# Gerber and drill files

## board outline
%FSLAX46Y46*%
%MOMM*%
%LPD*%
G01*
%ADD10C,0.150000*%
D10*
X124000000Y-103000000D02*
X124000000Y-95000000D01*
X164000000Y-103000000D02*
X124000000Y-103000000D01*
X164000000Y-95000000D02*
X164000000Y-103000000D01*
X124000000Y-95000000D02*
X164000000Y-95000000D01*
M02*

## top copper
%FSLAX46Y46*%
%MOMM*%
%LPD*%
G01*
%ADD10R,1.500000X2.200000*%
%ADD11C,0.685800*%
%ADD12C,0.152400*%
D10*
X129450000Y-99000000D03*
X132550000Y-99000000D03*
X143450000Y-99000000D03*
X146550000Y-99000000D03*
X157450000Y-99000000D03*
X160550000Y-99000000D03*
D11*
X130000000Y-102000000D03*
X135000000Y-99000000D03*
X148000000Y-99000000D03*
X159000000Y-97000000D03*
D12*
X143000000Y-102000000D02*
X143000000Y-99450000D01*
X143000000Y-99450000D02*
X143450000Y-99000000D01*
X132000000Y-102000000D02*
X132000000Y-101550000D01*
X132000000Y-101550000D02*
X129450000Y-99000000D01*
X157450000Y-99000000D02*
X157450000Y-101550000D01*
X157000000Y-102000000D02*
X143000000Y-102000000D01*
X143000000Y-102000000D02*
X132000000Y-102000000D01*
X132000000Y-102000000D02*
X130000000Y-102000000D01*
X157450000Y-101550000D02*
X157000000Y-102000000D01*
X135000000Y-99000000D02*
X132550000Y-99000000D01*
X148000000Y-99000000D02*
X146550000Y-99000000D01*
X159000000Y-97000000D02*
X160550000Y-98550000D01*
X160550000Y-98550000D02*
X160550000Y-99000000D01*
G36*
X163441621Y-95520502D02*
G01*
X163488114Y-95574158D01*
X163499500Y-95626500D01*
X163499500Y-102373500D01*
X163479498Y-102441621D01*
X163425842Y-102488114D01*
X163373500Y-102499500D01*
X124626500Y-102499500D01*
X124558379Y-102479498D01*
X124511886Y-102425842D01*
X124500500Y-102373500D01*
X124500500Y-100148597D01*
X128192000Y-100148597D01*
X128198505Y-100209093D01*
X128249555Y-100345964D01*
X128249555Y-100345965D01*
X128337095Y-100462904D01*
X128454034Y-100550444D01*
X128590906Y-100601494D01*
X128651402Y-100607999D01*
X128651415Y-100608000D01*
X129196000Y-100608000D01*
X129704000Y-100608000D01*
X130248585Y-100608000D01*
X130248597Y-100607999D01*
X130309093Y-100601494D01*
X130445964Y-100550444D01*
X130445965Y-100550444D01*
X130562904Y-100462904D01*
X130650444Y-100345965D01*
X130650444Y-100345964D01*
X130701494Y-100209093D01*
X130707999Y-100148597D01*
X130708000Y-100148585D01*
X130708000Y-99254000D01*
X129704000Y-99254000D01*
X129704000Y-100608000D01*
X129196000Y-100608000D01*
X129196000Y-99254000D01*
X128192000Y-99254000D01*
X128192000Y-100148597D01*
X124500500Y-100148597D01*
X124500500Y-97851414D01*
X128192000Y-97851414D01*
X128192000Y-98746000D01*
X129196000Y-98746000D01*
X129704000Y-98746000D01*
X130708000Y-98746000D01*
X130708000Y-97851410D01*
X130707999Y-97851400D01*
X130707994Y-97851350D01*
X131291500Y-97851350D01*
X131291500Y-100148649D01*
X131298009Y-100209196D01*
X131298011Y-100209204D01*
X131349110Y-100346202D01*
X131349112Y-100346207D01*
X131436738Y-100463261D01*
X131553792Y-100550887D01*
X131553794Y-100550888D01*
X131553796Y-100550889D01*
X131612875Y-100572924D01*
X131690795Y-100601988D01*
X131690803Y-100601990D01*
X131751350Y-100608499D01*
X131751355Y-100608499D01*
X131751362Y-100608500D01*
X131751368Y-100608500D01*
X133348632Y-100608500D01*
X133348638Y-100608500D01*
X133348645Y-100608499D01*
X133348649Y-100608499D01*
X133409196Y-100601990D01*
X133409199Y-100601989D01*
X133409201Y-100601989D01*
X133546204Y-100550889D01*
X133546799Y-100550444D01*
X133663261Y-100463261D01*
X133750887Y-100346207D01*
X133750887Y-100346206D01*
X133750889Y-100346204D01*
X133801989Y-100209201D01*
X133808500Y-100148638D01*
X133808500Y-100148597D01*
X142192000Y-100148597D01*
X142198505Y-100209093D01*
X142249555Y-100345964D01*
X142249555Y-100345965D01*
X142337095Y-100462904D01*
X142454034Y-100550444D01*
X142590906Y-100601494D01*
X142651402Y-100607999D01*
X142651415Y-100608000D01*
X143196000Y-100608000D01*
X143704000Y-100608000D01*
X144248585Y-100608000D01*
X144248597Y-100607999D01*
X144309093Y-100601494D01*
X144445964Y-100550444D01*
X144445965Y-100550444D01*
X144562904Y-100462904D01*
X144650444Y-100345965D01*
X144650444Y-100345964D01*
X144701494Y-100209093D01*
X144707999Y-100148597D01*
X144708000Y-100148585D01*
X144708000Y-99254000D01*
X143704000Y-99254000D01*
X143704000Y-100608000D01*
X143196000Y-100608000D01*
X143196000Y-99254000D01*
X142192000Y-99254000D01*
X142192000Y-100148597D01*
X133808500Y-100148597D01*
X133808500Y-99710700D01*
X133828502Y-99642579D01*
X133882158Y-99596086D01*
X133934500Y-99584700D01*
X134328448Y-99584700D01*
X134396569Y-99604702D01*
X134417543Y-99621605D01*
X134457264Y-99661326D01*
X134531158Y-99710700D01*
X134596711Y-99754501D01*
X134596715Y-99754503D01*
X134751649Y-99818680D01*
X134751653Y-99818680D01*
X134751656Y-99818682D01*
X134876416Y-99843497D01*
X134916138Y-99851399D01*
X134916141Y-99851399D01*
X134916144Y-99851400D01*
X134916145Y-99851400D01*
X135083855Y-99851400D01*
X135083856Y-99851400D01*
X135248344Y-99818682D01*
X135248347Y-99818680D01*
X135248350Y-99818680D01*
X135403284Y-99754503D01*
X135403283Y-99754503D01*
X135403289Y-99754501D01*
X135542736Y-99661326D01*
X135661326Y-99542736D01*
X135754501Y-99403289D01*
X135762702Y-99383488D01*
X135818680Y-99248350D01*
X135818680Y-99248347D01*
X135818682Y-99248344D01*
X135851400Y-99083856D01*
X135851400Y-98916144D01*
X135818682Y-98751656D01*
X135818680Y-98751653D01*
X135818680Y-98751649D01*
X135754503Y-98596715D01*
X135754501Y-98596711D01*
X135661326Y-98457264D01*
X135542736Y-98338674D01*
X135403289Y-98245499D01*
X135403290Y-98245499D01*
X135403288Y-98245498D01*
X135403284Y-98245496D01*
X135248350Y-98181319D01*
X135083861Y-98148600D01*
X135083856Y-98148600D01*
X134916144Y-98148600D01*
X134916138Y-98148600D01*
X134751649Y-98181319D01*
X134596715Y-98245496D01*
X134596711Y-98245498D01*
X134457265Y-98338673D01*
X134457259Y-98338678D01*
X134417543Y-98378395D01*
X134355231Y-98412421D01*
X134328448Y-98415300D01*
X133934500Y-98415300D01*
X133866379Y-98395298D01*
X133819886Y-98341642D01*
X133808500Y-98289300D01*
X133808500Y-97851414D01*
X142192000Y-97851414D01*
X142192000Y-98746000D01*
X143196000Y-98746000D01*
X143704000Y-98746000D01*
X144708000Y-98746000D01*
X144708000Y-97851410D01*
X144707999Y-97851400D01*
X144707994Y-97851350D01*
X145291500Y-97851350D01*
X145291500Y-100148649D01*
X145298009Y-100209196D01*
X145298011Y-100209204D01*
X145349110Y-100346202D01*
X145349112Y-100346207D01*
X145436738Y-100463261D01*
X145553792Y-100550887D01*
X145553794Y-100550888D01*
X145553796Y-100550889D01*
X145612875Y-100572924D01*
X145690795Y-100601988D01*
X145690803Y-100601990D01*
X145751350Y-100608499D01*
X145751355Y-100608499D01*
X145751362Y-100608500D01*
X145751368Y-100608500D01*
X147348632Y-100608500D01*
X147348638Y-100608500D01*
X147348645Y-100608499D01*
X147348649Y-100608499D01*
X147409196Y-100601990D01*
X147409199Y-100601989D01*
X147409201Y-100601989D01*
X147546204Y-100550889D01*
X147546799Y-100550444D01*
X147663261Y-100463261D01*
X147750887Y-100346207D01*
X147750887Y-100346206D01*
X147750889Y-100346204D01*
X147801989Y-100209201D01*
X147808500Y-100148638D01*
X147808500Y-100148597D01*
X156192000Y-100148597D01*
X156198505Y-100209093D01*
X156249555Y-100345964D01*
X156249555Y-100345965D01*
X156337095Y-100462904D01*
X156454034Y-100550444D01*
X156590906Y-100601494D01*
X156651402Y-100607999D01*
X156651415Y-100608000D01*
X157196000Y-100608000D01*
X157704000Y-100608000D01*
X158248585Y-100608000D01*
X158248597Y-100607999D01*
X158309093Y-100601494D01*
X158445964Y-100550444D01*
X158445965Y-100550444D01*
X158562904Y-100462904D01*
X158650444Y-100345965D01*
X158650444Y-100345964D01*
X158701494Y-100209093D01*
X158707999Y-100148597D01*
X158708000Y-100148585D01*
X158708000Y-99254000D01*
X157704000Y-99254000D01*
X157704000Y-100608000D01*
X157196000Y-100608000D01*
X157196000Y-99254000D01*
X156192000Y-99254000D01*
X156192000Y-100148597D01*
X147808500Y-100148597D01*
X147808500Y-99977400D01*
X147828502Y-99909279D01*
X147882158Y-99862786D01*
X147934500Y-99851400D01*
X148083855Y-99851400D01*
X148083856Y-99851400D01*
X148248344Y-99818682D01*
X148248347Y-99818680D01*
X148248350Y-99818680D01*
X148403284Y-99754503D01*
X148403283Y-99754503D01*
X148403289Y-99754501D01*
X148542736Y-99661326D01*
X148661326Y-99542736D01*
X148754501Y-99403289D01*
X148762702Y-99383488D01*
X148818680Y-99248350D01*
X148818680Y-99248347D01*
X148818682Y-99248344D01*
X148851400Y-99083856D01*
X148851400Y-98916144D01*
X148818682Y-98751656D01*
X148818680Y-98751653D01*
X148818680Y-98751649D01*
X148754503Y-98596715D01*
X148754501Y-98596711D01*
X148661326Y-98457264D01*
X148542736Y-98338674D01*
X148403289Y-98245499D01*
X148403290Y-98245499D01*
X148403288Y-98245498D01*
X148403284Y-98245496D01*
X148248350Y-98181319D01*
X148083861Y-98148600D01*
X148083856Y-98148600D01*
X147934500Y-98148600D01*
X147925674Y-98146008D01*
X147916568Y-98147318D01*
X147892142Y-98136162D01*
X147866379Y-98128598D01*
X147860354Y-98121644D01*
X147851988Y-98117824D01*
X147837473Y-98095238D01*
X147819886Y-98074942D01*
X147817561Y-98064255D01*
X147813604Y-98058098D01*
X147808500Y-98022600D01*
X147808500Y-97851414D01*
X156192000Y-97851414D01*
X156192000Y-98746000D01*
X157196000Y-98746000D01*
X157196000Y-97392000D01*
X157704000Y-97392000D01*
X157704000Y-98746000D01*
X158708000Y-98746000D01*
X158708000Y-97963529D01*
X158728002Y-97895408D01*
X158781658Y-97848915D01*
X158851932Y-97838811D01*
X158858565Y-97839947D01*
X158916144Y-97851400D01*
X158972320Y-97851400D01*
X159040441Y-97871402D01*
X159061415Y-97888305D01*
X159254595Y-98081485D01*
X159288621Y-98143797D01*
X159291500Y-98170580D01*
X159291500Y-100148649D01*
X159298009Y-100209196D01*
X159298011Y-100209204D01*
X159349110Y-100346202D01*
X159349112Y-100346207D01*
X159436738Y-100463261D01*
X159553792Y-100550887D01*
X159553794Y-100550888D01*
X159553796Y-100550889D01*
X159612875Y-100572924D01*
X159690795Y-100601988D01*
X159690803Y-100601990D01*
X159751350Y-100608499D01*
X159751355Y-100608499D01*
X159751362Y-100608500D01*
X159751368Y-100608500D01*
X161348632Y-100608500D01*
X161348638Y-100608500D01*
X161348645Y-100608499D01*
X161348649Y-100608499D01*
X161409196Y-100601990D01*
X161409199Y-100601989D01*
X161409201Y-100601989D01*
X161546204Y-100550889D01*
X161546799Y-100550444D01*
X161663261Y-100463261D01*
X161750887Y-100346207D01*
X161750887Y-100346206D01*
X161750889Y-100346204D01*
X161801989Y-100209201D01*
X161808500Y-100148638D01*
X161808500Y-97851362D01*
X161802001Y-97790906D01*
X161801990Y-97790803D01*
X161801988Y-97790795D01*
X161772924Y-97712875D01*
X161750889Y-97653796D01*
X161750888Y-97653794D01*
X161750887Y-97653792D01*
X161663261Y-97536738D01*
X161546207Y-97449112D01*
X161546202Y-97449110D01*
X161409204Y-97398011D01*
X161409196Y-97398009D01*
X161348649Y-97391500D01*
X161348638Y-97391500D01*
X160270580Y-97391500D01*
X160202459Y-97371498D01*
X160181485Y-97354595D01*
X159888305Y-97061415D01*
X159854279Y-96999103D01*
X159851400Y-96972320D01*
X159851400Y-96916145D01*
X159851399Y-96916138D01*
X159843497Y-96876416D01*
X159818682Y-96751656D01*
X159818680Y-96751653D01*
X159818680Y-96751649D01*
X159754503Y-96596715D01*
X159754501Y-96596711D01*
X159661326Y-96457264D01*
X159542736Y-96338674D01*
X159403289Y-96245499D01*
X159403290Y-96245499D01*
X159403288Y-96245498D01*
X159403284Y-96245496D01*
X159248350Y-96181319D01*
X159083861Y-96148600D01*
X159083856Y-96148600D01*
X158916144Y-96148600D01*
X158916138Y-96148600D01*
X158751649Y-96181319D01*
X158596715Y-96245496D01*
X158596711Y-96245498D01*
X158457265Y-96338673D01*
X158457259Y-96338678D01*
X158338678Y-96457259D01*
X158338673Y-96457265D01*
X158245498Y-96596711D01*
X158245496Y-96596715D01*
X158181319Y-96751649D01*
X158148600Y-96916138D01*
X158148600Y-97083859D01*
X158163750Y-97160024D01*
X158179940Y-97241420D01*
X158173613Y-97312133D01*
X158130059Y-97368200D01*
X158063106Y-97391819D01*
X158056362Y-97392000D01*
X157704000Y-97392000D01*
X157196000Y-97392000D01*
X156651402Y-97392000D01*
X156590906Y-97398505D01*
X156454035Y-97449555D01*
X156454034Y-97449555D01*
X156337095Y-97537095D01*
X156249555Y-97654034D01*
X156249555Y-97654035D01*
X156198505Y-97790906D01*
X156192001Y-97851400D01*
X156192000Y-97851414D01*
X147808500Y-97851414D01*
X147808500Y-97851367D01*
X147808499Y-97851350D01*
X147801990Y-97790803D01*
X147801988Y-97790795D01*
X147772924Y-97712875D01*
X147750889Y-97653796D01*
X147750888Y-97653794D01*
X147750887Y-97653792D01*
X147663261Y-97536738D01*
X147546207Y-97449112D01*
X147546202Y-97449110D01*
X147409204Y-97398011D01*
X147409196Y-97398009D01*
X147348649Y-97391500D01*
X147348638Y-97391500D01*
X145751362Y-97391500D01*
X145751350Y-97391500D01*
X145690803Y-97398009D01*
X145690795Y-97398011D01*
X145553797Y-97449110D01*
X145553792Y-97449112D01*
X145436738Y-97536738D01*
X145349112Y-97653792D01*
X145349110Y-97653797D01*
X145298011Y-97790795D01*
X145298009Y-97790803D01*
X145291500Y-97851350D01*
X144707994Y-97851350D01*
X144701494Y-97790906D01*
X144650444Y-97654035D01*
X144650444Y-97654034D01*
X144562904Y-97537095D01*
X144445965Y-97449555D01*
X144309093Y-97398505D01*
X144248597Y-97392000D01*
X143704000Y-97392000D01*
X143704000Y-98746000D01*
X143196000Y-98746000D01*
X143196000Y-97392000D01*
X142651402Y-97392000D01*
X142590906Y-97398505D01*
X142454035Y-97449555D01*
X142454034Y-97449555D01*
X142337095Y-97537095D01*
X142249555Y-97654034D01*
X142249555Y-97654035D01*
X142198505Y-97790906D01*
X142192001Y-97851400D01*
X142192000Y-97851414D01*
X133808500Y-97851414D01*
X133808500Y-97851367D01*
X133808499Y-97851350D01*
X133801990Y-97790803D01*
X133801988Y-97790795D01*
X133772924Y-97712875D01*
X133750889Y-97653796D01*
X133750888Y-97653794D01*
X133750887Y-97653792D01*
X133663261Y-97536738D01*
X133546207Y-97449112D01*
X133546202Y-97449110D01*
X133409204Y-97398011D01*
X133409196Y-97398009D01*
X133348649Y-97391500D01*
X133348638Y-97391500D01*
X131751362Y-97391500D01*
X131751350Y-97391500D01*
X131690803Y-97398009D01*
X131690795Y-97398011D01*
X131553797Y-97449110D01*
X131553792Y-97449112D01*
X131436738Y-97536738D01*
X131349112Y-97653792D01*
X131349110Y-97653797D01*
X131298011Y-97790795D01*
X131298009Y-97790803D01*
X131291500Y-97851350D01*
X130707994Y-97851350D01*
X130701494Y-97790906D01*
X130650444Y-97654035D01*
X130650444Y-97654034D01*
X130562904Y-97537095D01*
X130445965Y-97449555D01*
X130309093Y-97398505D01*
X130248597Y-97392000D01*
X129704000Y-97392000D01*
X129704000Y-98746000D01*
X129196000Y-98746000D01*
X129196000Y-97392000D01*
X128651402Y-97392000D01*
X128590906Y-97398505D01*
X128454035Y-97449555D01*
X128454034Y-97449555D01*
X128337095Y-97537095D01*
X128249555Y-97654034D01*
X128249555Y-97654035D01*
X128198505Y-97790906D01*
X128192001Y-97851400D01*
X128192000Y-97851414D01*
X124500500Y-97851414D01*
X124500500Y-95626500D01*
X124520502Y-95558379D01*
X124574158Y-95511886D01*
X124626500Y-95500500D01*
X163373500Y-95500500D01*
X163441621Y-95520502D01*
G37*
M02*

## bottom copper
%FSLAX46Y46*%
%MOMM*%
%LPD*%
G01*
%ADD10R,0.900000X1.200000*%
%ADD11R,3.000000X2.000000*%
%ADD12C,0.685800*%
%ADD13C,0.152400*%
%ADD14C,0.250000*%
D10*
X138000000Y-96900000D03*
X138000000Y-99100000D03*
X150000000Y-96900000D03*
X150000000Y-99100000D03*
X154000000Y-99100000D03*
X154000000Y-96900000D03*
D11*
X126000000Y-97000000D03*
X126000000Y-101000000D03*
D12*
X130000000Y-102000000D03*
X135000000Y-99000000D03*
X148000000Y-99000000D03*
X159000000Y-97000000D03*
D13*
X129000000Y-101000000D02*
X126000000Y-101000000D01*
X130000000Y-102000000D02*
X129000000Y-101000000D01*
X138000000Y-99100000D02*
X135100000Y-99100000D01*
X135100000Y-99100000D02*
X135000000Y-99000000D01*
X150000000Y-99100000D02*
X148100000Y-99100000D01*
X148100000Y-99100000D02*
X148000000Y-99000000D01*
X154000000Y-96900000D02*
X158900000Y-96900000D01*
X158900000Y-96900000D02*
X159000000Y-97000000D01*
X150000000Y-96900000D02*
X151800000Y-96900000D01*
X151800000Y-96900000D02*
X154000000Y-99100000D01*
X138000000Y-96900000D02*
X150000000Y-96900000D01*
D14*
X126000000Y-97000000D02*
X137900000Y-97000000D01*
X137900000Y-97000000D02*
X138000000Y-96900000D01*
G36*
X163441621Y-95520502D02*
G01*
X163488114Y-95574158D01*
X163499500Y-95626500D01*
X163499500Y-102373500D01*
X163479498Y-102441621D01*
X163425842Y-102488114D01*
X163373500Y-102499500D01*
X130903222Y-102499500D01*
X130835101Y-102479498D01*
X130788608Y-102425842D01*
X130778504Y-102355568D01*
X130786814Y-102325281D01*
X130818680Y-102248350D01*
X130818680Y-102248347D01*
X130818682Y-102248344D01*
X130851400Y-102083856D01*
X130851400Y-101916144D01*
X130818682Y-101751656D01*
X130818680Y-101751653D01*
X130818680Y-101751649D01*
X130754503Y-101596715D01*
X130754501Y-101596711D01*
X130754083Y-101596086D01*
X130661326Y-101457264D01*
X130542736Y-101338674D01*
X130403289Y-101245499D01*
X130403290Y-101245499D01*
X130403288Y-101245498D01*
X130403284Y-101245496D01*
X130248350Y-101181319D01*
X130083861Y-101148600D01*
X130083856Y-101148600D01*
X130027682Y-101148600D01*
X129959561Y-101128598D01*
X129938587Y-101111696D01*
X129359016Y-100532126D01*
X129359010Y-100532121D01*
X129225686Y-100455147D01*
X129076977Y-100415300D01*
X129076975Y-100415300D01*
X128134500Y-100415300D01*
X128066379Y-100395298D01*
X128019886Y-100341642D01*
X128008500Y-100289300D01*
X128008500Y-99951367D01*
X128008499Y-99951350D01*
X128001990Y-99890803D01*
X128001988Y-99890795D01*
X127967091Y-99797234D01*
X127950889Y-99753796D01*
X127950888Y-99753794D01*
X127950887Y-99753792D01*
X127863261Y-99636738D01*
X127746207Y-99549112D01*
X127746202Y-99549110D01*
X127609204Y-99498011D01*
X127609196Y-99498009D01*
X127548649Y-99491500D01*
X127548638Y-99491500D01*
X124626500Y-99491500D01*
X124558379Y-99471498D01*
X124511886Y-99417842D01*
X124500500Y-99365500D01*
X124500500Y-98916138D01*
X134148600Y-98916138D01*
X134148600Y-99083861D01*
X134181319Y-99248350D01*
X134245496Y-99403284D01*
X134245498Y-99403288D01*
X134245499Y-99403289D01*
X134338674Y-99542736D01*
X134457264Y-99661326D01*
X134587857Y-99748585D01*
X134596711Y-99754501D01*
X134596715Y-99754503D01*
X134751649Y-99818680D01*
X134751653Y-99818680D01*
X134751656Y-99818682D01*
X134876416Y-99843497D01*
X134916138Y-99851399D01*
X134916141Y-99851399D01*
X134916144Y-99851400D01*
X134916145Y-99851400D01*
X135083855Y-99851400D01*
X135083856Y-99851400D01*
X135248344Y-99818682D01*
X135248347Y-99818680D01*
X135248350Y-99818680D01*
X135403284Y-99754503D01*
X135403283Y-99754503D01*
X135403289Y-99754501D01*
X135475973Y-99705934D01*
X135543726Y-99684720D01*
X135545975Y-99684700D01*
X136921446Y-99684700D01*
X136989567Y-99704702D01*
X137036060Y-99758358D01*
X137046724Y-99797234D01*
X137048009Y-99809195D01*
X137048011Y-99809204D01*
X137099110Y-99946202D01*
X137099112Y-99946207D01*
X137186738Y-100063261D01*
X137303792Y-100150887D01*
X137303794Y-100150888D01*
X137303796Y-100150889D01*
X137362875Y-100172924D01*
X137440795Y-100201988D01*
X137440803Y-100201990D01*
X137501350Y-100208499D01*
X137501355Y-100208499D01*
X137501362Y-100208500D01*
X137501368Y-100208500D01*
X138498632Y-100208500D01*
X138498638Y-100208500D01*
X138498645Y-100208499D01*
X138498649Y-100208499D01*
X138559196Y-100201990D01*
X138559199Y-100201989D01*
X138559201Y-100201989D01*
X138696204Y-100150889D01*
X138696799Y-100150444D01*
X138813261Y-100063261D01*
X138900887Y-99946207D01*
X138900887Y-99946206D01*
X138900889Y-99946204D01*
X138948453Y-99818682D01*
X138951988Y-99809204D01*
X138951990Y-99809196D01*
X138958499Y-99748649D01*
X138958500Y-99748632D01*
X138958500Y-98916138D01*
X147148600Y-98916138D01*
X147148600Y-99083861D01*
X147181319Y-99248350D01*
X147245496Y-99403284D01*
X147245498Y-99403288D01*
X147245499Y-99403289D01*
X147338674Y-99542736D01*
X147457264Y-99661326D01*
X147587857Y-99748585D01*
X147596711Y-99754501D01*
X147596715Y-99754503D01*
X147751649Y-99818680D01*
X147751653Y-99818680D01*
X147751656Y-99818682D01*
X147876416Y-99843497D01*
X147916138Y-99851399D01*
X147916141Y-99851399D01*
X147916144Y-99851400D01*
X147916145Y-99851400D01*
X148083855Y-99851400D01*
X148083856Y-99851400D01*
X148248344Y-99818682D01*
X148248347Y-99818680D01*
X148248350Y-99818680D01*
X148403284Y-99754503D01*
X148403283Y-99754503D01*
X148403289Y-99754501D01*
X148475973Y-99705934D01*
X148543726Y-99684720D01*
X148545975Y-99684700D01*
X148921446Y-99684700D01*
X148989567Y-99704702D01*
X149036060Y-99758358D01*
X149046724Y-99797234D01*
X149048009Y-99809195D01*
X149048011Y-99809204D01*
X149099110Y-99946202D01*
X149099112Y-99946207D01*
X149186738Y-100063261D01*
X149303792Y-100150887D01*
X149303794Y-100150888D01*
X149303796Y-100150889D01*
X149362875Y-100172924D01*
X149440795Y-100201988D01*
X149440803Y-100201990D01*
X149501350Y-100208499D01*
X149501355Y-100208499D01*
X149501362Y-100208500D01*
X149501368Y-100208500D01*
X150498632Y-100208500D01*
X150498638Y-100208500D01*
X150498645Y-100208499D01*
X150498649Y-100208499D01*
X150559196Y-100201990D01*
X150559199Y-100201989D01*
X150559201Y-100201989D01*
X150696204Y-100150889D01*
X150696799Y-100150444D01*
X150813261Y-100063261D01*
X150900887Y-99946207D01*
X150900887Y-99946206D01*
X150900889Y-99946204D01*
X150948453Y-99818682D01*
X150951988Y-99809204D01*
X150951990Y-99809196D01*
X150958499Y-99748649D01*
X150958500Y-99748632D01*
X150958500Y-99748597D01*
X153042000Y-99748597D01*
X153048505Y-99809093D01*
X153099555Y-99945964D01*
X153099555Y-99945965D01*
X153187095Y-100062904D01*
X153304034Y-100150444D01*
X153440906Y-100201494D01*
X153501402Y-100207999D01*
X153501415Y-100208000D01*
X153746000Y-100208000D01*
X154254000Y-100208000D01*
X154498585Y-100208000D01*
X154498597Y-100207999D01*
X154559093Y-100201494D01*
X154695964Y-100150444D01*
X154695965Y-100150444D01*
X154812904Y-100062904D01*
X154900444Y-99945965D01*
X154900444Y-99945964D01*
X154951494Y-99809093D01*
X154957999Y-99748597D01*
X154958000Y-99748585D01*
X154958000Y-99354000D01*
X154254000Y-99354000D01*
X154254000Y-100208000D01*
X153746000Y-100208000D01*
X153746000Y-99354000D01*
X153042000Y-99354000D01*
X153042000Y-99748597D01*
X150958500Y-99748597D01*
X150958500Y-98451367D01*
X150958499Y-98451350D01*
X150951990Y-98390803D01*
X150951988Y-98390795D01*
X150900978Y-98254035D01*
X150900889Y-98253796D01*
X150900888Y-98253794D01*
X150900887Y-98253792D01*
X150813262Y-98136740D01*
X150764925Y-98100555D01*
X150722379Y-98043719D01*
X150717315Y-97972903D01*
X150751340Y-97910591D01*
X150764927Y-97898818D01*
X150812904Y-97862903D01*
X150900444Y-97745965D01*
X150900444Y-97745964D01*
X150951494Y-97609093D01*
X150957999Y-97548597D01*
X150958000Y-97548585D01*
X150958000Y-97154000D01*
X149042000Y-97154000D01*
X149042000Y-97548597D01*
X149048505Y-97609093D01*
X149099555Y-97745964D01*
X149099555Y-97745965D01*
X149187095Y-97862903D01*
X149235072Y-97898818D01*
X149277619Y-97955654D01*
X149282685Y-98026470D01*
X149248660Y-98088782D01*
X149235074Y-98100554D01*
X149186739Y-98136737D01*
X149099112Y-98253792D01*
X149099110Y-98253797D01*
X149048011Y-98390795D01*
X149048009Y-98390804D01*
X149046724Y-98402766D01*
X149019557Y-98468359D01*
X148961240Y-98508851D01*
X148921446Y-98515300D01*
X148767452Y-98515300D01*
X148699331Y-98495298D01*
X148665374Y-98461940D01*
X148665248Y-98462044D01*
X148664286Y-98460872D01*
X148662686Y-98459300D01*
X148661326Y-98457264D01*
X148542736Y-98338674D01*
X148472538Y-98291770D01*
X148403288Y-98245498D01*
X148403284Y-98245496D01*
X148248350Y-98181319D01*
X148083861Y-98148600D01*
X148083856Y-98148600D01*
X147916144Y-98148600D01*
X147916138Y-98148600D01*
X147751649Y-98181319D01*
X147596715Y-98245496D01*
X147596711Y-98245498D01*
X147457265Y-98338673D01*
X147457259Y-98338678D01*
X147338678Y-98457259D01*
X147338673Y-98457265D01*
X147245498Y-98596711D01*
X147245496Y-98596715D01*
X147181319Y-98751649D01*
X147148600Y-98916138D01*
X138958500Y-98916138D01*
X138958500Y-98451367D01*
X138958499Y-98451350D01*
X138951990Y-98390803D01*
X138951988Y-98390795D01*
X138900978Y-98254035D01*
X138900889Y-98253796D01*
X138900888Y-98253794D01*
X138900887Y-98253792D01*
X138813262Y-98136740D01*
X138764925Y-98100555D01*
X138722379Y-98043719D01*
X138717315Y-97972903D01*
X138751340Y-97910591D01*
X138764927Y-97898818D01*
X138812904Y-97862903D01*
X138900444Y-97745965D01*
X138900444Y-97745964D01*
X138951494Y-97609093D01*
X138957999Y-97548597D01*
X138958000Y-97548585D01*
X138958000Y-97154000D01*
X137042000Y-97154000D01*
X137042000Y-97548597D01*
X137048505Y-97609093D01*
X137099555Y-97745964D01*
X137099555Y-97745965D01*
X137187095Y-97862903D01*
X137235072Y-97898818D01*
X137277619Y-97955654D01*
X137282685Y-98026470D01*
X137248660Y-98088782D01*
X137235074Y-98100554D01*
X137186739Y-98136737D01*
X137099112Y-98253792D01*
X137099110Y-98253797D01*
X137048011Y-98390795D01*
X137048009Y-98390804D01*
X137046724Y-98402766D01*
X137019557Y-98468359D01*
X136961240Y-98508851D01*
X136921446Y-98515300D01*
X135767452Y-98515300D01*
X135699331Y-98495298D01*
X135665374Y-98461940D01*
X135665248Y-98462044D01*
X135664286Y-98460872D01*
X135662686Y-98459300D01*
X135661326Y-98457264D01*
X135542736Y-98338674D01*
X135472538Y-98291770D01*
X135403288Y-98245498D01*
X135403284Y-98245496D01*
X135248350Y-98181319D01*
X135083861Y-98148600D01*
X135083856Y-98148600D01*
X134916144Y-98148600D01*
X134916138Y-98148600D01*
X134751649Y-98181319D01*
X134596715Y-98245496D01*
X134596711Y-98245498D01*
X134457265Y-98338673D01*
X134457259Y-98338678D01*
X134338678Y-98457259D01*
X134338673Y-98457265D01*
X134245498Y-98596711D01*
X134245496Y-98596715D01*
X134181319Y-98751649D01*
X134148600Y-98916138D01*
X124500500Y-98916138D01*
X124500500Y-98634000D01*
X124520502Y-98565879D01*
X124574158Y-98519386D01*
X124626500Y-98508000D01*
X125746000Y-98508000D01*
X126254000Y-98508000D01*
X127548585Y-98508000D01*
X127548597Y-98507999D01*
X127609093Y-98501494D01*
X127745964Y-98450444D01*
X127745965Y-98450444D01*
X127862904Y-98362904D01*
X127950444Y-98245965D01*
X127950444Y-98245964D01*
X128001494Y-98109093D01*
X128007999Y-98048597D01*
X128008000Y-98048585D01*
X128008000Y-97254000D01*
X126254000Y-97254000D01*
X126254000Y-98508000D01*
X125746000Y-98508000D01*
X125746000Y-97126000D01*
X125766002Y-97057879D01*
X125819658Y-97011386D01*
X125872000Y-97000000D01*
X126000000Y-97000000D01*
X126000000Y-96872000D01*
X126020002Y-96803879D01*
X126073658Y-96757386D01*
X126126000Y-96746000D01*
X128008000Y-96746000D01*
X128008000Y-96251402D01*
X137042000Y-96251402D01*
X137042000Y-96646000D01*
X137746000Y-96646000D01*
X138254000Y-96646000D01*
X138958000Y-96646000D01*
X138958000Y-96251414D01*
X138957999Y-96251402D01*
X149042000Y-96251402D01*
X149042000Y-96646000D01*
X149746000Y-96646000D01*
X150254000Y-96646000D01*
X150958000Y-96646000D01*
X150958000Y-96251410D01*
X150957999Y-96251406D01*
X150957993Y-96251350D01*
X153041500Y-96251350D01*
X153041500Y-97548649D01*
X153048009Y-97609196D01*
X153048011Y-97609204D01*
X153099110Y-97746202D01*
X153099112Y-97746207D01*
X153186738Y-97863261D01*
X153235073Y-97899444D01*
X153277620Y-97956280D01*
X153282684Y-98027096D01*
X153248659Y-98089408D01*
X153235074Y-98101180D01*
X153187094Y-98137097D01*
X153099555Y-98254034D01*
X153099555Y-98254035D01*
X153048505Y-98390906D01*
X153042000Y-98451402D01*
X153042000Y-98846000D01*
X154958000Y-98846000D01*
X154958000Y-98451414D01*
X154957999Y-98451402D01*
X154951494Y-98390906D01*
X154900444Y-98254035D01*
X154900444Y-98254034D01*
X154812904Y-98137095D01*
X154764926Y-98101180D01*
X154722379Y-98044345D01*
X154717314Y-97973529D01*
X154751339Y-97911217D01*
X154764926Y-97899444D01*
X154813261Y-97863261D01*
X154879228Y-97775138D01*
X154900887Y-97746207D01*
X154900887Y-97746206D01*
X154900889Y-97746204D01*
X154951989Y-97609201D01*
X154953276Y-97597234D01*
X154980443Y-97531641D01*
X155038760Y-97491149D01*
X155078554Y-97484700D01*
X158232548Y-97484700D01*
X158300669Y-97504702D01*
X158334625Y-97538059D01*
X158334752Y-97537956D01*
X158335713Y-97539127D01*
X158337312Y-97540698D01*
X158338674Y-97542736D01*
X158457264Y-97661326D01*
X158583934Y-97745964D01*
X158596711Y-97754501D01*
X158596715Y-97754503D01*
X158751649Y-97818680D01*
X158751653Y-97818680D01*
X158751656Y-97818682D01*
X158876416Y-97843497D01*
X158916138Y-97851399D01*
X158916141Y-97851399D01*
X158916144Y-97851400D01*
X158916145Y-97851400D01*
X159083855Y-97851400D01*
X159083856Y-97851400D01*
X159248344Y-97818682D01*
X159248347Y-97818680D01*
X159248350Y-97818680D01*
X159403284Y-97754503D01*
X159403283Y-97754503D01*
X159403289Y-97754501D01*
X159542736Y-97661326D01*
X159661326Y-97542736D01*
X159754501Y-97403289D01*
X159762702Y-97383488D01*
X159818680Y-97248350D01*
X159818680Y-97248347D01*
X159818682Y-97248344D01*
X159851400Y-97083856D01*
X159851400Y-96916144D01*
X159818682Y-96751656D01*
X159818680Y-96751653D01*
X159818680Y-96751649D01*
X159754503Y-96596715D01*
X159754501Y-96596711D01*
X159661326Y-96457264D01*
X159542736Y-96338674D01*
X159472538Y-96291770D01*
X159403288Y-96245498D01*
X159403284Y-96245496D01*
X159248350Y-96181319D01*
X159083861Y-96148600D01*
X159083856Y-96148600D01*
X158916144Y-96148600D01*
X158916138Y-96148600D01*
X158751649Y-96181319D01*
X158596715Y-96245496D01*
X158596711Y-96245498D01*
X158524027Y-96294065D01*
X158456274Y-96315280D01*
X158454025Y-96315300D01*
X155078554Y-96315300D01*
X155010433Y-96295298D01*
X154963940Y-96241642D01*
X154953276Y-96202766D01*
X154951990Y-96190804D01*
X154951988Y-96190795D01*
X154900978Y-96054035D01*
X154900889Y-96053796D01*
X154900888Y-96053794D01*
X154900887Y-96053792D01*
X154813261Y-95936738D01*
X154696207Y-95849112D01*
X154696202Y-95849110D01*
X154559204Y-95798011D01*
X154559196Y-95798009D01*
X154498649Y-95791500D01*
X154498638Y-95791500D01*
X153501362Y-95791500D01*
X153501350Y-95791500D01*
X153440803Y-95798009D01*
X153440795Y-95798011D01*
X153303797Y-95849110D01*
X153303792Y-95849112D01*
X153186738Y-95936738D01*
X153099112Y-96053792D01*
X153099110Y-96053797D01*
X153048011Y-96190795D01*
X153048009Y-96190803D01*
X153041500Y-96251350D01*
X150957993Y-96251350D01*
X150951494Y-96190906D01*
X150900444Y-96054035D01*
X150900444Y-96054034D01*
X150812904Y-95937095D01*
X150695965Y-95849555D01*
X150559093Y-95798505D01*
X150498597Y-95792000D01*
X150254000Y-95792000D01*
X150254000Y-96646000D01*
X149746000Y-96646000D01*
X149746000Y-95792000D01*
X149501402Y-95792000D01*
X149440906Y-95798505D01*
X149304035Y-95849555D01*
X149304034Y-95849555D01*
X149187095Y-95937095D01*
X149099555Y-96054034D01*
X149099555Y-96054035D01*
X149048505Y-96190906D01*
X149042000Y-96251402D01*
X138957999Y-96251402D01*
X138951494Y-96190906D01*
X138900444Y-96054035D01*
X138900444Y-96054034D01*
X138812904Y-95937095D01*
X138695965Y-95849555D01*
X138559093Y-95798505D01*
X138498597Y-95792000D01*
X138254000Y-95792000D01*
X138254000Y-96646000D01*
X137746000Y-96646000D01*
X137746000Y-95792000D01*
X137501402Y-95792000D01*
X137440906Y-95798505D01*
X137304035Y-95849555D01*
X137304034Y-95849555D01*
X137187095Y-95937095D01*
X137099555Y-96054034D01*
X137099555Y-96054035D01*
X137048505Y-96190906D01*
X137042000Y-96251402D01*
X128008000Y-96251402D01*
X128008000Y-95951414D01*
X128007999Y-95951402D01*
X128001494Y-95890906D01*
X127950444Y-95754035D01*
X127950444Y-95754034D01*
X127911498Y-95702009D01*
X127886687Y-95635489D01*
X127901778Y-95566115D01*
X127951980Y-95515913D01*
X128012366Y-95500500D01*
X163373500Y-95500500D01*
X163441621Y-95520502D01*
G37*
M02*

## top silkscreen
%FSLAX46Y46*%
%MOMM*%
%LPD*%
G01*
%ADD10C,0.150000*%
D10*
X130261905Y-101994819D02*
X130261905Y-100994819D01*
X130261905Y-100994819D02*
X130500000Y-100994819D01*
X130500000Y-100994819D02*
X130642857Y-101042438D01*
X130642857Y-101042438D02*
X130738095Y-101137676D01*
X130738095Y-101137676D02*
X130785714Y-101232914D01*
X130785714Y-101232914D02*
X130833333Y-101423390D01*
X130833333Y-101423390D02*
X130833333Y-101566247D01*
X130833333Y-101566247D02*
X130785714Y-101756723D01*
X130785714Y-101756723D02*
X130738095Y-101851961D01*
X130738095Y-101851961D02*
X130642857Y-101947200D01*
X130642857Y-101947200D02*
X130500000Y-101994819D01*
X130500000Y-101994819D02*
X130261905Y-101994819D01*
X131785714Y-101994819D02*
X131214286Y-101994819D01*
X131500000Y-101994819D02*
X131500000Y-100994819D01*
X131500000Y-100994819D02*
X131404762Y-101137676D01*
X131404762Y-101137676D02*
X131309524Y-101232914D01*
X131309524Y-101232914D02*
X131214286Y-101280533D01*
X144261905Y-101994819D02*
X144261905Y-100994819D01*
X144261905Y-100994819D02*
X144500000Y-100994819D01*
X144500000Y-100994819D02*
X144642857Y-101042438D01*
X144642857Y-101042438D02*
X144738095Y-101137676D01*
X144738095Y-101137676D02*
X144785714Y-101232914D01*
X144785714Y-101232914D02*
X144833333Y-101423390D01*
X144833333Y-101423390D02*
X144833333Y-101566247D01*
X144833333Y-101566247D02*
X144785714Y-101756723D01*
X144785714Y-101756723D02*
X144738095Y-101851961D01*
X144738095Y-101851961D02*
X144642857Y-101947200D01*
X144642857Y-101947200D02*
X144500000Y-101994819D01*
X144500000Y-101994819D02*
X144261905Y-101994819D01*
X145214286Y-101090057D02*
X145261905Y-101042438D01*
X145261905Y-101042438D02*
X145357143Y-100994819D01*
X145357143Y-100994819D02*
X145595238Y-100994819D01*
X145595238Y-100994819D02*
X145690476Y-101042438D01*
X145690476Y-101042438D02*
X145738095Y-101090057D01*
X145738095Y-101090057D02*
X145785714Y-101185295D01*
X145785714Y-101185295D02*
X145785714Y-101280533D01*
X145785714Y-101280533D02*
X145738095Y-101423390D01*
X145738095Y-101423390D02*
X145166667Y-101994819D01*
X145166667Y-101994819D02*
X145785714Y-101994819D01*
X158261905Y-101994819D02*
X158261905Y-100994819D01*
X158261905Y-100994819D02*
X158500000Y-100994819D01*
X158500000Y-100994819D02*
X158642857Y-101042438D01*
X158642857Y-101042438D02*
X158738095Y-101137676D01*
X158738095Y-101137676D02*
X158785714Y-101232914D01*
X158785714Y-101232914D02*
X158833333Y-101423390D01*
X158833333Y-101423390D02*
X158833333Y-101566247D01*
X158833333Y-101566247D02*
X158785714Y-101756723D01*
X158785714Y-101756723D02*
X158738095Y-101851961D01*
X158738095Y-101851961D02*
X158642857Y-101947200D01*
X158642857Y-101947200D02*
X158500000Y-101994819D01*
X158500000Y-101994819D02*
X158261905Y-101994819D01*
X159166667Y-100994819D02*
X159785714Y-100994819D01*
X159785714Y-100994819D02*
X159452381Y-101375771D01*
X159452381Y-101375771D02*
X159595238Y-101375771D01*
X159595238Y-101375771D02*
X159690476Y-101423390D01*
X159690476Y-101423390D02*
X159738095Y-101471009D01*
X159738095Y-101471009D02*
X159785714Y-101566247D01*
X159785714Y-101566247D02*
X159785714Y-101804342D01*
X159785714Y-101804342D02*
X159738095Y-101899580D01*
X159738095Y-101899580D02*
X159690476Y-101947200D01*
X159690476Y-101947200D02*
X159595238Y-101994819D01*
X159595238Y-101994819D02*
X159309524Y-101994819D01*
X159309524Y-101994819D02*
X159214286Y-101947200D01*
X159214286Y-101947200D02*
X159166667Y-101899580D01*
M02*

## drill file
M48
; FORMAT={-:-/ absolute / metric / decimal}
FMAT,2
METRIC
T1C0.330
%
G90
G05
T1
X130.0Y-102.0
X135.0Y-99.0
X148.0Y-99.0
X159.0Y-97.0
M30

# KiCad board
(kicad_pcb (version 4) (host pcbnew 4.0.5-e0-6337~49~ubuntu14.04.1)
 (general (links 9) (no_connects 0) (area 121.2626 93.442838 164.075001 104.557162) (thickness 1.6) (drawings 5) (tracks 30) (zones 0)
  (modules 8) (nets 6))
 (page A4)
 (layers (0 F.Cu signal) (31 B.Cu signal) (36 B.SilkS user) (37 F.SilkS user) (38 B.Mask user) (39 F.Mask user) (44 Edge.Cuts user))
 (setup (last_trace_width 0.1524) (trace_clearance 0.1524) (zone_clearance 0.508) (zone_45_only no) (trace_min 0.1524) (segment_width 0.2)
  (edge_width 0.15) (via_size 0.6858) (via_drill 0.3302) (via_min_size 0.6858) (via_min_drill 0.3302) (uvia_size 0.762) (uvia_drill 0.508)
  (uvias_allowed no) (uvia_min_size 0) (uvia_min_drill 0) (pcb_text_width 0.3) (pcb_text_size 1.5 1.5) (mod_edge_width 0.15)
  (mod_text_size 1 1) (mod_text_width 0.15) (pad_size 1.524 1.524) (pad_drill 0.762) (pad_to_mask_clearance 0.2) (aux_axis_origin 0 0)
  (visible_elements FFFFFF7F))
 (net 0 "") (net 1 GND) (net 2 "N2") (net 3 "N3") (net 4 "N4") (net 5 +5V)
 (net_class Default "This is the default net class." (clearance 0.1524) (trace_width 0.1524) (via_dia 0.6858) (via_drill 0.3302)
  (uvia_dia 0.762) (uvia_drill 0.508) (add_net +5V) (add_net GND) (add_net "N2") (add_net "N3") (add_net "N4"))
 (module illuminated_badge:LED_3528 (layer F.Cu) (at 131 99)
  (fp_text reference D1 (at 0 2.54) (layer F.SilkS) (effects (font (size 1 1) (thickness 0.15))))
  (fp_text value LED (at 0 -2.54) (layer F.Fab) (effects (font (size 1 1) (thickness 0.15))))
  (pad 1 smd rect (at -1.55 0) (size 1.5 2.2) (layers F.Cu F.Mask) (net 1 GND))
  (pad 2 smd rect (at 1.55 0) (size 1.5 2.2) (layers F.Cu F.Mask) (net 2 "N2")))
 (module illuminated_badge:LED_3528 (layer F.Cu) (at 145 99)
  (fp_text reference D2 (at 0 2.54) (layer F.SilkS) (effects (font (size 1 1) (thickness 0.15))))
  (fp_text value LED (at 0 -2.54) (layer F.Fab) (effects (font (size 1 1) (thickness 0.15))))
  (pad 1 smd rect (at -1.55 0) (size 1.5 2.2) (layers F.Cu F.Mask) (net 1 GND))
  (pad 2 smd rect (at 1.55 0) (size 1.5 2.2) (layers F.Cu F.Mask) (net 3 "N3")))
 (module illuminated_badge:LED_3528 (layer F.Cu) (at 159 99)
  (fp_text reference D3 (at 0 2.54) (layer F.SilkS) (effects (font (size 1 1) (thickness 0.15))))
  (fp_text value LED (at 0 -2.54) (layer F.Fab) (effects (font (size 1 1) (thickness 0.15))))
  (pad 1 smd rect (at -1.55 0) (size 1.5 2.2) (layers F.Cu F.Mask) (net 1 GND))
  (pad 2 smd rect (at 1.55 0) (size 1.5 2.2) (layers F.Cu F.Mask) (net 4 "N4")))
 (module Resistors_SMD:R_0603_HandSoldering (layer B.Cu) (at 138 98 270)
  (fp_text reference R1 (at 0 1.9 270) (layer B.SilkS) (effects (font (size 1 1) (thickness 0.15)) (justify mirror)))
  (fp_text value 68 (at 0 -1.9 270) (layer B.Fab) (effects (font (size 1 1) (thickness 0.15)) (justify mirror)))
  (pad 1 smd rect (at -1.1 0 270) (size 1.2 0.9) (layers B.Cu B.Mask) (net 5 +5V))
  (pad 2 smd rect (at 1.1 0 270) (size 1.2 0.9) (layers B.Cu B.Mask) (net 2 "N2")))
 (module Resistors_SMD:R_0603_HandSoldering (layer B.Cu) (at 150 98 270)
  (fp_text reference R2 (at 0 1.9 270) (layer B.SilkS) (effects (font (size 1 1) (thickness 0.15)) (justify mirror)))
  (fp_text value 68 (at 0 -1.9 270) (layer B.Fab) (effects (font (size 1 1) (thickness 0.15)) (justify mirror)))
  (pad 1 smd rect (at -1.1 0 270) (size 1.2 0.9) (layers B.Cu B.Mask) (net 5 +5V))
  (pad 2 smd rect (at 1.1 0 270) (size 1.2 0.9) (layers B.Cu B.Mask) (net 3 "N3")))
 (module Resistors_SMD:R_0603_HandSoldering (layer B.Cu) (at 154 98 90)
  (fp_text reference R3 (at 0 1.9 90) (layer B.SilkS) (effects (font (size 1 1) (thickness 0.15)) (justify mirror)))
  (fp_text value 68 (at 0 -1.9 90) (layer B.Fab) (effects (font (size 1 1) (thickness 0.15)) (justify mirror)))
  (pad 1 smd rect (at -1.1 0 90) (size 1.2 0.9) (layers B.Cu B.Mask) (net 5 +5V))
  (pad 2 smd rect (at 1.1 0 90) (size 1.2 0.9) (layers B.Cu B.Mask) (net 4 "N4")))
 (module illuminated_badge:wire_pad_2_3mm (layer B.Cu) (at 126 97 90)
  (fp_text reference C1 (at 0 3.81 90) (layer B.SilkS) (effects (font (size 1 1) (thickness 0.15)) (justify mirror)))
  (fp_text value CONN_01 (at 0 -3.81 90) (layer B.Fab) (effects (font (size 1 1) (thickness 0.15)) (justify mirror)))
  (pad 1 smd rect (at 0 0 90) (size 2 3) (layers B.Cu B.Mask) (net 5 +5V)))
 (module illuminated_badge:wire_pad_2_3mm (layer B.Cu) (at 126 101 90)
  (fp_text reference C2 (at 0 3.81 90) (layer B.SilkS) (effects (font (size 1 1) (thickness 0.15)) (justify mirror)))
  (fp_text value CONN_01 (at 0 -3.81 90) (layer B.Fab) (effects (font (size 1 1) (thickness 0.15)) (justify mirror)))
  (pad 1 smd rect (at 0 0 90) (size 2 3) (layers B.Cu B.Mask) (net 1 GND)))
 (gr_line (start 124 103) (end 124 95) (angle 90) (layer Edge.Cuts) (width 0.15))
 (gr_line (start 164 103) (end 124 103) (angle 90) (layer Edge.Cuts) (width 0.15))
 (gr_line (start 164 95) (end 164 103) (angle 90) (layer Edge.Cuts) (width 0.15))
 (gr_line (start 124 95) (end 164 95) (angle 90) (layer Edge.Cuts) (width 0.15))
 (segment (start 143 102) (end 143 99.45) (width 0.1524) (layer F.Cu) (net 1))
 (segment (start 143 99.45) (end 143.45 99) (width 0.1524) (layer F.Cu) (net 1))
 (segment (start 132 102) (end 132 101.55) (width 0.1524) (layer F.Cu) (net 1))
 (segment (start 132 101.55) (end 129.45 99) (width 0.1524) (layer F.Cu) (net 1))
 (segment (start 157.45 99) (end 157.45 101.55) (width 0.1524) (layer F.Cu) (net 1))
 (segment (start 129 101) (end 126 101) (width 0.1524) (layer B.Cu) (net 1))
 (segment (start 130 102) (end 129 101) (width 0.1524) (layer B.Cu) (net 1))
 (via (at 130 102) (size 0.6858) (drill 0.3302) (layers F.Cu B.Cu) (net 1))
 (segment (start 157 102) (end 143 102) (width 0.1524) (layer F.Cu) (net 1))
 (segment (start 143 102) (end 132 102) (width 0.1524) (layer F.Cu) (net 1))
 (segment (start 132 102) (end 130 102) (width 0.1524) (layer F.Cu) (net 1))
 (segment (start 157.45 101.55) (end 157 102) (width 0.1524) (layer F.Cu) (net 1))
 (segment (start 138 99.1) (end 135.1 99.1) (width 0.1524) (layer B.Cu) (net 2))
 (segment (start 135 99) (end 132.55 99) (width 0.1524) (layer F.Cu) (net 2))
 (via (at 135 99) (size 0.6858) (drill 0.3302) (layers F.Cu B.Cu) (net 2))
 (segment (start 135.1 99.1) (end 135 99) (width 0.1524) (layer B.Cu) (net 2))
 (segment (start 150 99.1) (end 148.1 99.1) (width 0.1524) (layer B.Cu) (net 3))
 (segment (start 148 99) (end 146.55 99) (width 0.1524) (layer F.Cu) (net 3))
 (via (at 148 99) (size 0.6858) (drill 0.3302) (layers F.Cu B.Cu) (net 3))
 (segment (start 148.1 99.1) (end 148 99) (width 0.1524) (layer B.Cu) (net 3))
 (segment (start 154 96.9) (end 158.9 96.9) (width 0.1524) (layer B.Cu) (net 4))
 (segment (start 159 97) (end 160.55 98.55) (width 0.1524) (layer F.Cu) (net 4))
 (via (at 159 97) (size 0.6858) (drill 0.3302) (layers F.Cu B.Cu) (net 4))
 (segment (start 158.9 96.9) (end 159 97) (width 0.1524) (layer B.Cu) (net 4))
 (segment (start 160.55 98.55) (end 160.55 99) (width 0.1524) (layer F.Cu) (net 4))
 (segment (start 150 96.9) (end 151.8 96.9) (width 0.1524) (layer B.Cu) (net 5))
 (segment (start 151.8 96.9) (end 154 99.1) (width 0.1524) (layer B.Cu) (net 5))
 (segment (start 138 96.9) (end 150 96.9) (width 0.1524) (layer B.Cu) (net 5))
 (segment (start 126 97) (end 137.9 97) (width 0.25) (layer B.Cu) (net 5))
 (segment (start 137.9 97) (end 138 96.9) (width 0.25) (layer B.Cu) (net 5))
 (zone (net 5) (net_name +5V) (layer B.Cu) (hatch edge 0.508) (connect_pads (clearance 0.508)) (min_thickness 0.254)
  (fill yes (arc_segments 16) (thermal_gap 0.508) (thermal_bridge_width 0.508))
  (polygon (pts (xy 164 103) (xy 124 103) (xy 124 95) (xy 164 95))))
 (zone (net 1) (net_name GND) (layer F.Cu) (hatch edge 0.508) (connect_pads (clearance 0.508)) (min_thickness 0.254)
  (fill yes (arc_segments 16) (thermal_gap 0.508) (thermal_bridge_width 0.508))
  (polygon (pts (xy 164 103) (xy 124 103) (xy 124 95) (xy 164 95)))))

